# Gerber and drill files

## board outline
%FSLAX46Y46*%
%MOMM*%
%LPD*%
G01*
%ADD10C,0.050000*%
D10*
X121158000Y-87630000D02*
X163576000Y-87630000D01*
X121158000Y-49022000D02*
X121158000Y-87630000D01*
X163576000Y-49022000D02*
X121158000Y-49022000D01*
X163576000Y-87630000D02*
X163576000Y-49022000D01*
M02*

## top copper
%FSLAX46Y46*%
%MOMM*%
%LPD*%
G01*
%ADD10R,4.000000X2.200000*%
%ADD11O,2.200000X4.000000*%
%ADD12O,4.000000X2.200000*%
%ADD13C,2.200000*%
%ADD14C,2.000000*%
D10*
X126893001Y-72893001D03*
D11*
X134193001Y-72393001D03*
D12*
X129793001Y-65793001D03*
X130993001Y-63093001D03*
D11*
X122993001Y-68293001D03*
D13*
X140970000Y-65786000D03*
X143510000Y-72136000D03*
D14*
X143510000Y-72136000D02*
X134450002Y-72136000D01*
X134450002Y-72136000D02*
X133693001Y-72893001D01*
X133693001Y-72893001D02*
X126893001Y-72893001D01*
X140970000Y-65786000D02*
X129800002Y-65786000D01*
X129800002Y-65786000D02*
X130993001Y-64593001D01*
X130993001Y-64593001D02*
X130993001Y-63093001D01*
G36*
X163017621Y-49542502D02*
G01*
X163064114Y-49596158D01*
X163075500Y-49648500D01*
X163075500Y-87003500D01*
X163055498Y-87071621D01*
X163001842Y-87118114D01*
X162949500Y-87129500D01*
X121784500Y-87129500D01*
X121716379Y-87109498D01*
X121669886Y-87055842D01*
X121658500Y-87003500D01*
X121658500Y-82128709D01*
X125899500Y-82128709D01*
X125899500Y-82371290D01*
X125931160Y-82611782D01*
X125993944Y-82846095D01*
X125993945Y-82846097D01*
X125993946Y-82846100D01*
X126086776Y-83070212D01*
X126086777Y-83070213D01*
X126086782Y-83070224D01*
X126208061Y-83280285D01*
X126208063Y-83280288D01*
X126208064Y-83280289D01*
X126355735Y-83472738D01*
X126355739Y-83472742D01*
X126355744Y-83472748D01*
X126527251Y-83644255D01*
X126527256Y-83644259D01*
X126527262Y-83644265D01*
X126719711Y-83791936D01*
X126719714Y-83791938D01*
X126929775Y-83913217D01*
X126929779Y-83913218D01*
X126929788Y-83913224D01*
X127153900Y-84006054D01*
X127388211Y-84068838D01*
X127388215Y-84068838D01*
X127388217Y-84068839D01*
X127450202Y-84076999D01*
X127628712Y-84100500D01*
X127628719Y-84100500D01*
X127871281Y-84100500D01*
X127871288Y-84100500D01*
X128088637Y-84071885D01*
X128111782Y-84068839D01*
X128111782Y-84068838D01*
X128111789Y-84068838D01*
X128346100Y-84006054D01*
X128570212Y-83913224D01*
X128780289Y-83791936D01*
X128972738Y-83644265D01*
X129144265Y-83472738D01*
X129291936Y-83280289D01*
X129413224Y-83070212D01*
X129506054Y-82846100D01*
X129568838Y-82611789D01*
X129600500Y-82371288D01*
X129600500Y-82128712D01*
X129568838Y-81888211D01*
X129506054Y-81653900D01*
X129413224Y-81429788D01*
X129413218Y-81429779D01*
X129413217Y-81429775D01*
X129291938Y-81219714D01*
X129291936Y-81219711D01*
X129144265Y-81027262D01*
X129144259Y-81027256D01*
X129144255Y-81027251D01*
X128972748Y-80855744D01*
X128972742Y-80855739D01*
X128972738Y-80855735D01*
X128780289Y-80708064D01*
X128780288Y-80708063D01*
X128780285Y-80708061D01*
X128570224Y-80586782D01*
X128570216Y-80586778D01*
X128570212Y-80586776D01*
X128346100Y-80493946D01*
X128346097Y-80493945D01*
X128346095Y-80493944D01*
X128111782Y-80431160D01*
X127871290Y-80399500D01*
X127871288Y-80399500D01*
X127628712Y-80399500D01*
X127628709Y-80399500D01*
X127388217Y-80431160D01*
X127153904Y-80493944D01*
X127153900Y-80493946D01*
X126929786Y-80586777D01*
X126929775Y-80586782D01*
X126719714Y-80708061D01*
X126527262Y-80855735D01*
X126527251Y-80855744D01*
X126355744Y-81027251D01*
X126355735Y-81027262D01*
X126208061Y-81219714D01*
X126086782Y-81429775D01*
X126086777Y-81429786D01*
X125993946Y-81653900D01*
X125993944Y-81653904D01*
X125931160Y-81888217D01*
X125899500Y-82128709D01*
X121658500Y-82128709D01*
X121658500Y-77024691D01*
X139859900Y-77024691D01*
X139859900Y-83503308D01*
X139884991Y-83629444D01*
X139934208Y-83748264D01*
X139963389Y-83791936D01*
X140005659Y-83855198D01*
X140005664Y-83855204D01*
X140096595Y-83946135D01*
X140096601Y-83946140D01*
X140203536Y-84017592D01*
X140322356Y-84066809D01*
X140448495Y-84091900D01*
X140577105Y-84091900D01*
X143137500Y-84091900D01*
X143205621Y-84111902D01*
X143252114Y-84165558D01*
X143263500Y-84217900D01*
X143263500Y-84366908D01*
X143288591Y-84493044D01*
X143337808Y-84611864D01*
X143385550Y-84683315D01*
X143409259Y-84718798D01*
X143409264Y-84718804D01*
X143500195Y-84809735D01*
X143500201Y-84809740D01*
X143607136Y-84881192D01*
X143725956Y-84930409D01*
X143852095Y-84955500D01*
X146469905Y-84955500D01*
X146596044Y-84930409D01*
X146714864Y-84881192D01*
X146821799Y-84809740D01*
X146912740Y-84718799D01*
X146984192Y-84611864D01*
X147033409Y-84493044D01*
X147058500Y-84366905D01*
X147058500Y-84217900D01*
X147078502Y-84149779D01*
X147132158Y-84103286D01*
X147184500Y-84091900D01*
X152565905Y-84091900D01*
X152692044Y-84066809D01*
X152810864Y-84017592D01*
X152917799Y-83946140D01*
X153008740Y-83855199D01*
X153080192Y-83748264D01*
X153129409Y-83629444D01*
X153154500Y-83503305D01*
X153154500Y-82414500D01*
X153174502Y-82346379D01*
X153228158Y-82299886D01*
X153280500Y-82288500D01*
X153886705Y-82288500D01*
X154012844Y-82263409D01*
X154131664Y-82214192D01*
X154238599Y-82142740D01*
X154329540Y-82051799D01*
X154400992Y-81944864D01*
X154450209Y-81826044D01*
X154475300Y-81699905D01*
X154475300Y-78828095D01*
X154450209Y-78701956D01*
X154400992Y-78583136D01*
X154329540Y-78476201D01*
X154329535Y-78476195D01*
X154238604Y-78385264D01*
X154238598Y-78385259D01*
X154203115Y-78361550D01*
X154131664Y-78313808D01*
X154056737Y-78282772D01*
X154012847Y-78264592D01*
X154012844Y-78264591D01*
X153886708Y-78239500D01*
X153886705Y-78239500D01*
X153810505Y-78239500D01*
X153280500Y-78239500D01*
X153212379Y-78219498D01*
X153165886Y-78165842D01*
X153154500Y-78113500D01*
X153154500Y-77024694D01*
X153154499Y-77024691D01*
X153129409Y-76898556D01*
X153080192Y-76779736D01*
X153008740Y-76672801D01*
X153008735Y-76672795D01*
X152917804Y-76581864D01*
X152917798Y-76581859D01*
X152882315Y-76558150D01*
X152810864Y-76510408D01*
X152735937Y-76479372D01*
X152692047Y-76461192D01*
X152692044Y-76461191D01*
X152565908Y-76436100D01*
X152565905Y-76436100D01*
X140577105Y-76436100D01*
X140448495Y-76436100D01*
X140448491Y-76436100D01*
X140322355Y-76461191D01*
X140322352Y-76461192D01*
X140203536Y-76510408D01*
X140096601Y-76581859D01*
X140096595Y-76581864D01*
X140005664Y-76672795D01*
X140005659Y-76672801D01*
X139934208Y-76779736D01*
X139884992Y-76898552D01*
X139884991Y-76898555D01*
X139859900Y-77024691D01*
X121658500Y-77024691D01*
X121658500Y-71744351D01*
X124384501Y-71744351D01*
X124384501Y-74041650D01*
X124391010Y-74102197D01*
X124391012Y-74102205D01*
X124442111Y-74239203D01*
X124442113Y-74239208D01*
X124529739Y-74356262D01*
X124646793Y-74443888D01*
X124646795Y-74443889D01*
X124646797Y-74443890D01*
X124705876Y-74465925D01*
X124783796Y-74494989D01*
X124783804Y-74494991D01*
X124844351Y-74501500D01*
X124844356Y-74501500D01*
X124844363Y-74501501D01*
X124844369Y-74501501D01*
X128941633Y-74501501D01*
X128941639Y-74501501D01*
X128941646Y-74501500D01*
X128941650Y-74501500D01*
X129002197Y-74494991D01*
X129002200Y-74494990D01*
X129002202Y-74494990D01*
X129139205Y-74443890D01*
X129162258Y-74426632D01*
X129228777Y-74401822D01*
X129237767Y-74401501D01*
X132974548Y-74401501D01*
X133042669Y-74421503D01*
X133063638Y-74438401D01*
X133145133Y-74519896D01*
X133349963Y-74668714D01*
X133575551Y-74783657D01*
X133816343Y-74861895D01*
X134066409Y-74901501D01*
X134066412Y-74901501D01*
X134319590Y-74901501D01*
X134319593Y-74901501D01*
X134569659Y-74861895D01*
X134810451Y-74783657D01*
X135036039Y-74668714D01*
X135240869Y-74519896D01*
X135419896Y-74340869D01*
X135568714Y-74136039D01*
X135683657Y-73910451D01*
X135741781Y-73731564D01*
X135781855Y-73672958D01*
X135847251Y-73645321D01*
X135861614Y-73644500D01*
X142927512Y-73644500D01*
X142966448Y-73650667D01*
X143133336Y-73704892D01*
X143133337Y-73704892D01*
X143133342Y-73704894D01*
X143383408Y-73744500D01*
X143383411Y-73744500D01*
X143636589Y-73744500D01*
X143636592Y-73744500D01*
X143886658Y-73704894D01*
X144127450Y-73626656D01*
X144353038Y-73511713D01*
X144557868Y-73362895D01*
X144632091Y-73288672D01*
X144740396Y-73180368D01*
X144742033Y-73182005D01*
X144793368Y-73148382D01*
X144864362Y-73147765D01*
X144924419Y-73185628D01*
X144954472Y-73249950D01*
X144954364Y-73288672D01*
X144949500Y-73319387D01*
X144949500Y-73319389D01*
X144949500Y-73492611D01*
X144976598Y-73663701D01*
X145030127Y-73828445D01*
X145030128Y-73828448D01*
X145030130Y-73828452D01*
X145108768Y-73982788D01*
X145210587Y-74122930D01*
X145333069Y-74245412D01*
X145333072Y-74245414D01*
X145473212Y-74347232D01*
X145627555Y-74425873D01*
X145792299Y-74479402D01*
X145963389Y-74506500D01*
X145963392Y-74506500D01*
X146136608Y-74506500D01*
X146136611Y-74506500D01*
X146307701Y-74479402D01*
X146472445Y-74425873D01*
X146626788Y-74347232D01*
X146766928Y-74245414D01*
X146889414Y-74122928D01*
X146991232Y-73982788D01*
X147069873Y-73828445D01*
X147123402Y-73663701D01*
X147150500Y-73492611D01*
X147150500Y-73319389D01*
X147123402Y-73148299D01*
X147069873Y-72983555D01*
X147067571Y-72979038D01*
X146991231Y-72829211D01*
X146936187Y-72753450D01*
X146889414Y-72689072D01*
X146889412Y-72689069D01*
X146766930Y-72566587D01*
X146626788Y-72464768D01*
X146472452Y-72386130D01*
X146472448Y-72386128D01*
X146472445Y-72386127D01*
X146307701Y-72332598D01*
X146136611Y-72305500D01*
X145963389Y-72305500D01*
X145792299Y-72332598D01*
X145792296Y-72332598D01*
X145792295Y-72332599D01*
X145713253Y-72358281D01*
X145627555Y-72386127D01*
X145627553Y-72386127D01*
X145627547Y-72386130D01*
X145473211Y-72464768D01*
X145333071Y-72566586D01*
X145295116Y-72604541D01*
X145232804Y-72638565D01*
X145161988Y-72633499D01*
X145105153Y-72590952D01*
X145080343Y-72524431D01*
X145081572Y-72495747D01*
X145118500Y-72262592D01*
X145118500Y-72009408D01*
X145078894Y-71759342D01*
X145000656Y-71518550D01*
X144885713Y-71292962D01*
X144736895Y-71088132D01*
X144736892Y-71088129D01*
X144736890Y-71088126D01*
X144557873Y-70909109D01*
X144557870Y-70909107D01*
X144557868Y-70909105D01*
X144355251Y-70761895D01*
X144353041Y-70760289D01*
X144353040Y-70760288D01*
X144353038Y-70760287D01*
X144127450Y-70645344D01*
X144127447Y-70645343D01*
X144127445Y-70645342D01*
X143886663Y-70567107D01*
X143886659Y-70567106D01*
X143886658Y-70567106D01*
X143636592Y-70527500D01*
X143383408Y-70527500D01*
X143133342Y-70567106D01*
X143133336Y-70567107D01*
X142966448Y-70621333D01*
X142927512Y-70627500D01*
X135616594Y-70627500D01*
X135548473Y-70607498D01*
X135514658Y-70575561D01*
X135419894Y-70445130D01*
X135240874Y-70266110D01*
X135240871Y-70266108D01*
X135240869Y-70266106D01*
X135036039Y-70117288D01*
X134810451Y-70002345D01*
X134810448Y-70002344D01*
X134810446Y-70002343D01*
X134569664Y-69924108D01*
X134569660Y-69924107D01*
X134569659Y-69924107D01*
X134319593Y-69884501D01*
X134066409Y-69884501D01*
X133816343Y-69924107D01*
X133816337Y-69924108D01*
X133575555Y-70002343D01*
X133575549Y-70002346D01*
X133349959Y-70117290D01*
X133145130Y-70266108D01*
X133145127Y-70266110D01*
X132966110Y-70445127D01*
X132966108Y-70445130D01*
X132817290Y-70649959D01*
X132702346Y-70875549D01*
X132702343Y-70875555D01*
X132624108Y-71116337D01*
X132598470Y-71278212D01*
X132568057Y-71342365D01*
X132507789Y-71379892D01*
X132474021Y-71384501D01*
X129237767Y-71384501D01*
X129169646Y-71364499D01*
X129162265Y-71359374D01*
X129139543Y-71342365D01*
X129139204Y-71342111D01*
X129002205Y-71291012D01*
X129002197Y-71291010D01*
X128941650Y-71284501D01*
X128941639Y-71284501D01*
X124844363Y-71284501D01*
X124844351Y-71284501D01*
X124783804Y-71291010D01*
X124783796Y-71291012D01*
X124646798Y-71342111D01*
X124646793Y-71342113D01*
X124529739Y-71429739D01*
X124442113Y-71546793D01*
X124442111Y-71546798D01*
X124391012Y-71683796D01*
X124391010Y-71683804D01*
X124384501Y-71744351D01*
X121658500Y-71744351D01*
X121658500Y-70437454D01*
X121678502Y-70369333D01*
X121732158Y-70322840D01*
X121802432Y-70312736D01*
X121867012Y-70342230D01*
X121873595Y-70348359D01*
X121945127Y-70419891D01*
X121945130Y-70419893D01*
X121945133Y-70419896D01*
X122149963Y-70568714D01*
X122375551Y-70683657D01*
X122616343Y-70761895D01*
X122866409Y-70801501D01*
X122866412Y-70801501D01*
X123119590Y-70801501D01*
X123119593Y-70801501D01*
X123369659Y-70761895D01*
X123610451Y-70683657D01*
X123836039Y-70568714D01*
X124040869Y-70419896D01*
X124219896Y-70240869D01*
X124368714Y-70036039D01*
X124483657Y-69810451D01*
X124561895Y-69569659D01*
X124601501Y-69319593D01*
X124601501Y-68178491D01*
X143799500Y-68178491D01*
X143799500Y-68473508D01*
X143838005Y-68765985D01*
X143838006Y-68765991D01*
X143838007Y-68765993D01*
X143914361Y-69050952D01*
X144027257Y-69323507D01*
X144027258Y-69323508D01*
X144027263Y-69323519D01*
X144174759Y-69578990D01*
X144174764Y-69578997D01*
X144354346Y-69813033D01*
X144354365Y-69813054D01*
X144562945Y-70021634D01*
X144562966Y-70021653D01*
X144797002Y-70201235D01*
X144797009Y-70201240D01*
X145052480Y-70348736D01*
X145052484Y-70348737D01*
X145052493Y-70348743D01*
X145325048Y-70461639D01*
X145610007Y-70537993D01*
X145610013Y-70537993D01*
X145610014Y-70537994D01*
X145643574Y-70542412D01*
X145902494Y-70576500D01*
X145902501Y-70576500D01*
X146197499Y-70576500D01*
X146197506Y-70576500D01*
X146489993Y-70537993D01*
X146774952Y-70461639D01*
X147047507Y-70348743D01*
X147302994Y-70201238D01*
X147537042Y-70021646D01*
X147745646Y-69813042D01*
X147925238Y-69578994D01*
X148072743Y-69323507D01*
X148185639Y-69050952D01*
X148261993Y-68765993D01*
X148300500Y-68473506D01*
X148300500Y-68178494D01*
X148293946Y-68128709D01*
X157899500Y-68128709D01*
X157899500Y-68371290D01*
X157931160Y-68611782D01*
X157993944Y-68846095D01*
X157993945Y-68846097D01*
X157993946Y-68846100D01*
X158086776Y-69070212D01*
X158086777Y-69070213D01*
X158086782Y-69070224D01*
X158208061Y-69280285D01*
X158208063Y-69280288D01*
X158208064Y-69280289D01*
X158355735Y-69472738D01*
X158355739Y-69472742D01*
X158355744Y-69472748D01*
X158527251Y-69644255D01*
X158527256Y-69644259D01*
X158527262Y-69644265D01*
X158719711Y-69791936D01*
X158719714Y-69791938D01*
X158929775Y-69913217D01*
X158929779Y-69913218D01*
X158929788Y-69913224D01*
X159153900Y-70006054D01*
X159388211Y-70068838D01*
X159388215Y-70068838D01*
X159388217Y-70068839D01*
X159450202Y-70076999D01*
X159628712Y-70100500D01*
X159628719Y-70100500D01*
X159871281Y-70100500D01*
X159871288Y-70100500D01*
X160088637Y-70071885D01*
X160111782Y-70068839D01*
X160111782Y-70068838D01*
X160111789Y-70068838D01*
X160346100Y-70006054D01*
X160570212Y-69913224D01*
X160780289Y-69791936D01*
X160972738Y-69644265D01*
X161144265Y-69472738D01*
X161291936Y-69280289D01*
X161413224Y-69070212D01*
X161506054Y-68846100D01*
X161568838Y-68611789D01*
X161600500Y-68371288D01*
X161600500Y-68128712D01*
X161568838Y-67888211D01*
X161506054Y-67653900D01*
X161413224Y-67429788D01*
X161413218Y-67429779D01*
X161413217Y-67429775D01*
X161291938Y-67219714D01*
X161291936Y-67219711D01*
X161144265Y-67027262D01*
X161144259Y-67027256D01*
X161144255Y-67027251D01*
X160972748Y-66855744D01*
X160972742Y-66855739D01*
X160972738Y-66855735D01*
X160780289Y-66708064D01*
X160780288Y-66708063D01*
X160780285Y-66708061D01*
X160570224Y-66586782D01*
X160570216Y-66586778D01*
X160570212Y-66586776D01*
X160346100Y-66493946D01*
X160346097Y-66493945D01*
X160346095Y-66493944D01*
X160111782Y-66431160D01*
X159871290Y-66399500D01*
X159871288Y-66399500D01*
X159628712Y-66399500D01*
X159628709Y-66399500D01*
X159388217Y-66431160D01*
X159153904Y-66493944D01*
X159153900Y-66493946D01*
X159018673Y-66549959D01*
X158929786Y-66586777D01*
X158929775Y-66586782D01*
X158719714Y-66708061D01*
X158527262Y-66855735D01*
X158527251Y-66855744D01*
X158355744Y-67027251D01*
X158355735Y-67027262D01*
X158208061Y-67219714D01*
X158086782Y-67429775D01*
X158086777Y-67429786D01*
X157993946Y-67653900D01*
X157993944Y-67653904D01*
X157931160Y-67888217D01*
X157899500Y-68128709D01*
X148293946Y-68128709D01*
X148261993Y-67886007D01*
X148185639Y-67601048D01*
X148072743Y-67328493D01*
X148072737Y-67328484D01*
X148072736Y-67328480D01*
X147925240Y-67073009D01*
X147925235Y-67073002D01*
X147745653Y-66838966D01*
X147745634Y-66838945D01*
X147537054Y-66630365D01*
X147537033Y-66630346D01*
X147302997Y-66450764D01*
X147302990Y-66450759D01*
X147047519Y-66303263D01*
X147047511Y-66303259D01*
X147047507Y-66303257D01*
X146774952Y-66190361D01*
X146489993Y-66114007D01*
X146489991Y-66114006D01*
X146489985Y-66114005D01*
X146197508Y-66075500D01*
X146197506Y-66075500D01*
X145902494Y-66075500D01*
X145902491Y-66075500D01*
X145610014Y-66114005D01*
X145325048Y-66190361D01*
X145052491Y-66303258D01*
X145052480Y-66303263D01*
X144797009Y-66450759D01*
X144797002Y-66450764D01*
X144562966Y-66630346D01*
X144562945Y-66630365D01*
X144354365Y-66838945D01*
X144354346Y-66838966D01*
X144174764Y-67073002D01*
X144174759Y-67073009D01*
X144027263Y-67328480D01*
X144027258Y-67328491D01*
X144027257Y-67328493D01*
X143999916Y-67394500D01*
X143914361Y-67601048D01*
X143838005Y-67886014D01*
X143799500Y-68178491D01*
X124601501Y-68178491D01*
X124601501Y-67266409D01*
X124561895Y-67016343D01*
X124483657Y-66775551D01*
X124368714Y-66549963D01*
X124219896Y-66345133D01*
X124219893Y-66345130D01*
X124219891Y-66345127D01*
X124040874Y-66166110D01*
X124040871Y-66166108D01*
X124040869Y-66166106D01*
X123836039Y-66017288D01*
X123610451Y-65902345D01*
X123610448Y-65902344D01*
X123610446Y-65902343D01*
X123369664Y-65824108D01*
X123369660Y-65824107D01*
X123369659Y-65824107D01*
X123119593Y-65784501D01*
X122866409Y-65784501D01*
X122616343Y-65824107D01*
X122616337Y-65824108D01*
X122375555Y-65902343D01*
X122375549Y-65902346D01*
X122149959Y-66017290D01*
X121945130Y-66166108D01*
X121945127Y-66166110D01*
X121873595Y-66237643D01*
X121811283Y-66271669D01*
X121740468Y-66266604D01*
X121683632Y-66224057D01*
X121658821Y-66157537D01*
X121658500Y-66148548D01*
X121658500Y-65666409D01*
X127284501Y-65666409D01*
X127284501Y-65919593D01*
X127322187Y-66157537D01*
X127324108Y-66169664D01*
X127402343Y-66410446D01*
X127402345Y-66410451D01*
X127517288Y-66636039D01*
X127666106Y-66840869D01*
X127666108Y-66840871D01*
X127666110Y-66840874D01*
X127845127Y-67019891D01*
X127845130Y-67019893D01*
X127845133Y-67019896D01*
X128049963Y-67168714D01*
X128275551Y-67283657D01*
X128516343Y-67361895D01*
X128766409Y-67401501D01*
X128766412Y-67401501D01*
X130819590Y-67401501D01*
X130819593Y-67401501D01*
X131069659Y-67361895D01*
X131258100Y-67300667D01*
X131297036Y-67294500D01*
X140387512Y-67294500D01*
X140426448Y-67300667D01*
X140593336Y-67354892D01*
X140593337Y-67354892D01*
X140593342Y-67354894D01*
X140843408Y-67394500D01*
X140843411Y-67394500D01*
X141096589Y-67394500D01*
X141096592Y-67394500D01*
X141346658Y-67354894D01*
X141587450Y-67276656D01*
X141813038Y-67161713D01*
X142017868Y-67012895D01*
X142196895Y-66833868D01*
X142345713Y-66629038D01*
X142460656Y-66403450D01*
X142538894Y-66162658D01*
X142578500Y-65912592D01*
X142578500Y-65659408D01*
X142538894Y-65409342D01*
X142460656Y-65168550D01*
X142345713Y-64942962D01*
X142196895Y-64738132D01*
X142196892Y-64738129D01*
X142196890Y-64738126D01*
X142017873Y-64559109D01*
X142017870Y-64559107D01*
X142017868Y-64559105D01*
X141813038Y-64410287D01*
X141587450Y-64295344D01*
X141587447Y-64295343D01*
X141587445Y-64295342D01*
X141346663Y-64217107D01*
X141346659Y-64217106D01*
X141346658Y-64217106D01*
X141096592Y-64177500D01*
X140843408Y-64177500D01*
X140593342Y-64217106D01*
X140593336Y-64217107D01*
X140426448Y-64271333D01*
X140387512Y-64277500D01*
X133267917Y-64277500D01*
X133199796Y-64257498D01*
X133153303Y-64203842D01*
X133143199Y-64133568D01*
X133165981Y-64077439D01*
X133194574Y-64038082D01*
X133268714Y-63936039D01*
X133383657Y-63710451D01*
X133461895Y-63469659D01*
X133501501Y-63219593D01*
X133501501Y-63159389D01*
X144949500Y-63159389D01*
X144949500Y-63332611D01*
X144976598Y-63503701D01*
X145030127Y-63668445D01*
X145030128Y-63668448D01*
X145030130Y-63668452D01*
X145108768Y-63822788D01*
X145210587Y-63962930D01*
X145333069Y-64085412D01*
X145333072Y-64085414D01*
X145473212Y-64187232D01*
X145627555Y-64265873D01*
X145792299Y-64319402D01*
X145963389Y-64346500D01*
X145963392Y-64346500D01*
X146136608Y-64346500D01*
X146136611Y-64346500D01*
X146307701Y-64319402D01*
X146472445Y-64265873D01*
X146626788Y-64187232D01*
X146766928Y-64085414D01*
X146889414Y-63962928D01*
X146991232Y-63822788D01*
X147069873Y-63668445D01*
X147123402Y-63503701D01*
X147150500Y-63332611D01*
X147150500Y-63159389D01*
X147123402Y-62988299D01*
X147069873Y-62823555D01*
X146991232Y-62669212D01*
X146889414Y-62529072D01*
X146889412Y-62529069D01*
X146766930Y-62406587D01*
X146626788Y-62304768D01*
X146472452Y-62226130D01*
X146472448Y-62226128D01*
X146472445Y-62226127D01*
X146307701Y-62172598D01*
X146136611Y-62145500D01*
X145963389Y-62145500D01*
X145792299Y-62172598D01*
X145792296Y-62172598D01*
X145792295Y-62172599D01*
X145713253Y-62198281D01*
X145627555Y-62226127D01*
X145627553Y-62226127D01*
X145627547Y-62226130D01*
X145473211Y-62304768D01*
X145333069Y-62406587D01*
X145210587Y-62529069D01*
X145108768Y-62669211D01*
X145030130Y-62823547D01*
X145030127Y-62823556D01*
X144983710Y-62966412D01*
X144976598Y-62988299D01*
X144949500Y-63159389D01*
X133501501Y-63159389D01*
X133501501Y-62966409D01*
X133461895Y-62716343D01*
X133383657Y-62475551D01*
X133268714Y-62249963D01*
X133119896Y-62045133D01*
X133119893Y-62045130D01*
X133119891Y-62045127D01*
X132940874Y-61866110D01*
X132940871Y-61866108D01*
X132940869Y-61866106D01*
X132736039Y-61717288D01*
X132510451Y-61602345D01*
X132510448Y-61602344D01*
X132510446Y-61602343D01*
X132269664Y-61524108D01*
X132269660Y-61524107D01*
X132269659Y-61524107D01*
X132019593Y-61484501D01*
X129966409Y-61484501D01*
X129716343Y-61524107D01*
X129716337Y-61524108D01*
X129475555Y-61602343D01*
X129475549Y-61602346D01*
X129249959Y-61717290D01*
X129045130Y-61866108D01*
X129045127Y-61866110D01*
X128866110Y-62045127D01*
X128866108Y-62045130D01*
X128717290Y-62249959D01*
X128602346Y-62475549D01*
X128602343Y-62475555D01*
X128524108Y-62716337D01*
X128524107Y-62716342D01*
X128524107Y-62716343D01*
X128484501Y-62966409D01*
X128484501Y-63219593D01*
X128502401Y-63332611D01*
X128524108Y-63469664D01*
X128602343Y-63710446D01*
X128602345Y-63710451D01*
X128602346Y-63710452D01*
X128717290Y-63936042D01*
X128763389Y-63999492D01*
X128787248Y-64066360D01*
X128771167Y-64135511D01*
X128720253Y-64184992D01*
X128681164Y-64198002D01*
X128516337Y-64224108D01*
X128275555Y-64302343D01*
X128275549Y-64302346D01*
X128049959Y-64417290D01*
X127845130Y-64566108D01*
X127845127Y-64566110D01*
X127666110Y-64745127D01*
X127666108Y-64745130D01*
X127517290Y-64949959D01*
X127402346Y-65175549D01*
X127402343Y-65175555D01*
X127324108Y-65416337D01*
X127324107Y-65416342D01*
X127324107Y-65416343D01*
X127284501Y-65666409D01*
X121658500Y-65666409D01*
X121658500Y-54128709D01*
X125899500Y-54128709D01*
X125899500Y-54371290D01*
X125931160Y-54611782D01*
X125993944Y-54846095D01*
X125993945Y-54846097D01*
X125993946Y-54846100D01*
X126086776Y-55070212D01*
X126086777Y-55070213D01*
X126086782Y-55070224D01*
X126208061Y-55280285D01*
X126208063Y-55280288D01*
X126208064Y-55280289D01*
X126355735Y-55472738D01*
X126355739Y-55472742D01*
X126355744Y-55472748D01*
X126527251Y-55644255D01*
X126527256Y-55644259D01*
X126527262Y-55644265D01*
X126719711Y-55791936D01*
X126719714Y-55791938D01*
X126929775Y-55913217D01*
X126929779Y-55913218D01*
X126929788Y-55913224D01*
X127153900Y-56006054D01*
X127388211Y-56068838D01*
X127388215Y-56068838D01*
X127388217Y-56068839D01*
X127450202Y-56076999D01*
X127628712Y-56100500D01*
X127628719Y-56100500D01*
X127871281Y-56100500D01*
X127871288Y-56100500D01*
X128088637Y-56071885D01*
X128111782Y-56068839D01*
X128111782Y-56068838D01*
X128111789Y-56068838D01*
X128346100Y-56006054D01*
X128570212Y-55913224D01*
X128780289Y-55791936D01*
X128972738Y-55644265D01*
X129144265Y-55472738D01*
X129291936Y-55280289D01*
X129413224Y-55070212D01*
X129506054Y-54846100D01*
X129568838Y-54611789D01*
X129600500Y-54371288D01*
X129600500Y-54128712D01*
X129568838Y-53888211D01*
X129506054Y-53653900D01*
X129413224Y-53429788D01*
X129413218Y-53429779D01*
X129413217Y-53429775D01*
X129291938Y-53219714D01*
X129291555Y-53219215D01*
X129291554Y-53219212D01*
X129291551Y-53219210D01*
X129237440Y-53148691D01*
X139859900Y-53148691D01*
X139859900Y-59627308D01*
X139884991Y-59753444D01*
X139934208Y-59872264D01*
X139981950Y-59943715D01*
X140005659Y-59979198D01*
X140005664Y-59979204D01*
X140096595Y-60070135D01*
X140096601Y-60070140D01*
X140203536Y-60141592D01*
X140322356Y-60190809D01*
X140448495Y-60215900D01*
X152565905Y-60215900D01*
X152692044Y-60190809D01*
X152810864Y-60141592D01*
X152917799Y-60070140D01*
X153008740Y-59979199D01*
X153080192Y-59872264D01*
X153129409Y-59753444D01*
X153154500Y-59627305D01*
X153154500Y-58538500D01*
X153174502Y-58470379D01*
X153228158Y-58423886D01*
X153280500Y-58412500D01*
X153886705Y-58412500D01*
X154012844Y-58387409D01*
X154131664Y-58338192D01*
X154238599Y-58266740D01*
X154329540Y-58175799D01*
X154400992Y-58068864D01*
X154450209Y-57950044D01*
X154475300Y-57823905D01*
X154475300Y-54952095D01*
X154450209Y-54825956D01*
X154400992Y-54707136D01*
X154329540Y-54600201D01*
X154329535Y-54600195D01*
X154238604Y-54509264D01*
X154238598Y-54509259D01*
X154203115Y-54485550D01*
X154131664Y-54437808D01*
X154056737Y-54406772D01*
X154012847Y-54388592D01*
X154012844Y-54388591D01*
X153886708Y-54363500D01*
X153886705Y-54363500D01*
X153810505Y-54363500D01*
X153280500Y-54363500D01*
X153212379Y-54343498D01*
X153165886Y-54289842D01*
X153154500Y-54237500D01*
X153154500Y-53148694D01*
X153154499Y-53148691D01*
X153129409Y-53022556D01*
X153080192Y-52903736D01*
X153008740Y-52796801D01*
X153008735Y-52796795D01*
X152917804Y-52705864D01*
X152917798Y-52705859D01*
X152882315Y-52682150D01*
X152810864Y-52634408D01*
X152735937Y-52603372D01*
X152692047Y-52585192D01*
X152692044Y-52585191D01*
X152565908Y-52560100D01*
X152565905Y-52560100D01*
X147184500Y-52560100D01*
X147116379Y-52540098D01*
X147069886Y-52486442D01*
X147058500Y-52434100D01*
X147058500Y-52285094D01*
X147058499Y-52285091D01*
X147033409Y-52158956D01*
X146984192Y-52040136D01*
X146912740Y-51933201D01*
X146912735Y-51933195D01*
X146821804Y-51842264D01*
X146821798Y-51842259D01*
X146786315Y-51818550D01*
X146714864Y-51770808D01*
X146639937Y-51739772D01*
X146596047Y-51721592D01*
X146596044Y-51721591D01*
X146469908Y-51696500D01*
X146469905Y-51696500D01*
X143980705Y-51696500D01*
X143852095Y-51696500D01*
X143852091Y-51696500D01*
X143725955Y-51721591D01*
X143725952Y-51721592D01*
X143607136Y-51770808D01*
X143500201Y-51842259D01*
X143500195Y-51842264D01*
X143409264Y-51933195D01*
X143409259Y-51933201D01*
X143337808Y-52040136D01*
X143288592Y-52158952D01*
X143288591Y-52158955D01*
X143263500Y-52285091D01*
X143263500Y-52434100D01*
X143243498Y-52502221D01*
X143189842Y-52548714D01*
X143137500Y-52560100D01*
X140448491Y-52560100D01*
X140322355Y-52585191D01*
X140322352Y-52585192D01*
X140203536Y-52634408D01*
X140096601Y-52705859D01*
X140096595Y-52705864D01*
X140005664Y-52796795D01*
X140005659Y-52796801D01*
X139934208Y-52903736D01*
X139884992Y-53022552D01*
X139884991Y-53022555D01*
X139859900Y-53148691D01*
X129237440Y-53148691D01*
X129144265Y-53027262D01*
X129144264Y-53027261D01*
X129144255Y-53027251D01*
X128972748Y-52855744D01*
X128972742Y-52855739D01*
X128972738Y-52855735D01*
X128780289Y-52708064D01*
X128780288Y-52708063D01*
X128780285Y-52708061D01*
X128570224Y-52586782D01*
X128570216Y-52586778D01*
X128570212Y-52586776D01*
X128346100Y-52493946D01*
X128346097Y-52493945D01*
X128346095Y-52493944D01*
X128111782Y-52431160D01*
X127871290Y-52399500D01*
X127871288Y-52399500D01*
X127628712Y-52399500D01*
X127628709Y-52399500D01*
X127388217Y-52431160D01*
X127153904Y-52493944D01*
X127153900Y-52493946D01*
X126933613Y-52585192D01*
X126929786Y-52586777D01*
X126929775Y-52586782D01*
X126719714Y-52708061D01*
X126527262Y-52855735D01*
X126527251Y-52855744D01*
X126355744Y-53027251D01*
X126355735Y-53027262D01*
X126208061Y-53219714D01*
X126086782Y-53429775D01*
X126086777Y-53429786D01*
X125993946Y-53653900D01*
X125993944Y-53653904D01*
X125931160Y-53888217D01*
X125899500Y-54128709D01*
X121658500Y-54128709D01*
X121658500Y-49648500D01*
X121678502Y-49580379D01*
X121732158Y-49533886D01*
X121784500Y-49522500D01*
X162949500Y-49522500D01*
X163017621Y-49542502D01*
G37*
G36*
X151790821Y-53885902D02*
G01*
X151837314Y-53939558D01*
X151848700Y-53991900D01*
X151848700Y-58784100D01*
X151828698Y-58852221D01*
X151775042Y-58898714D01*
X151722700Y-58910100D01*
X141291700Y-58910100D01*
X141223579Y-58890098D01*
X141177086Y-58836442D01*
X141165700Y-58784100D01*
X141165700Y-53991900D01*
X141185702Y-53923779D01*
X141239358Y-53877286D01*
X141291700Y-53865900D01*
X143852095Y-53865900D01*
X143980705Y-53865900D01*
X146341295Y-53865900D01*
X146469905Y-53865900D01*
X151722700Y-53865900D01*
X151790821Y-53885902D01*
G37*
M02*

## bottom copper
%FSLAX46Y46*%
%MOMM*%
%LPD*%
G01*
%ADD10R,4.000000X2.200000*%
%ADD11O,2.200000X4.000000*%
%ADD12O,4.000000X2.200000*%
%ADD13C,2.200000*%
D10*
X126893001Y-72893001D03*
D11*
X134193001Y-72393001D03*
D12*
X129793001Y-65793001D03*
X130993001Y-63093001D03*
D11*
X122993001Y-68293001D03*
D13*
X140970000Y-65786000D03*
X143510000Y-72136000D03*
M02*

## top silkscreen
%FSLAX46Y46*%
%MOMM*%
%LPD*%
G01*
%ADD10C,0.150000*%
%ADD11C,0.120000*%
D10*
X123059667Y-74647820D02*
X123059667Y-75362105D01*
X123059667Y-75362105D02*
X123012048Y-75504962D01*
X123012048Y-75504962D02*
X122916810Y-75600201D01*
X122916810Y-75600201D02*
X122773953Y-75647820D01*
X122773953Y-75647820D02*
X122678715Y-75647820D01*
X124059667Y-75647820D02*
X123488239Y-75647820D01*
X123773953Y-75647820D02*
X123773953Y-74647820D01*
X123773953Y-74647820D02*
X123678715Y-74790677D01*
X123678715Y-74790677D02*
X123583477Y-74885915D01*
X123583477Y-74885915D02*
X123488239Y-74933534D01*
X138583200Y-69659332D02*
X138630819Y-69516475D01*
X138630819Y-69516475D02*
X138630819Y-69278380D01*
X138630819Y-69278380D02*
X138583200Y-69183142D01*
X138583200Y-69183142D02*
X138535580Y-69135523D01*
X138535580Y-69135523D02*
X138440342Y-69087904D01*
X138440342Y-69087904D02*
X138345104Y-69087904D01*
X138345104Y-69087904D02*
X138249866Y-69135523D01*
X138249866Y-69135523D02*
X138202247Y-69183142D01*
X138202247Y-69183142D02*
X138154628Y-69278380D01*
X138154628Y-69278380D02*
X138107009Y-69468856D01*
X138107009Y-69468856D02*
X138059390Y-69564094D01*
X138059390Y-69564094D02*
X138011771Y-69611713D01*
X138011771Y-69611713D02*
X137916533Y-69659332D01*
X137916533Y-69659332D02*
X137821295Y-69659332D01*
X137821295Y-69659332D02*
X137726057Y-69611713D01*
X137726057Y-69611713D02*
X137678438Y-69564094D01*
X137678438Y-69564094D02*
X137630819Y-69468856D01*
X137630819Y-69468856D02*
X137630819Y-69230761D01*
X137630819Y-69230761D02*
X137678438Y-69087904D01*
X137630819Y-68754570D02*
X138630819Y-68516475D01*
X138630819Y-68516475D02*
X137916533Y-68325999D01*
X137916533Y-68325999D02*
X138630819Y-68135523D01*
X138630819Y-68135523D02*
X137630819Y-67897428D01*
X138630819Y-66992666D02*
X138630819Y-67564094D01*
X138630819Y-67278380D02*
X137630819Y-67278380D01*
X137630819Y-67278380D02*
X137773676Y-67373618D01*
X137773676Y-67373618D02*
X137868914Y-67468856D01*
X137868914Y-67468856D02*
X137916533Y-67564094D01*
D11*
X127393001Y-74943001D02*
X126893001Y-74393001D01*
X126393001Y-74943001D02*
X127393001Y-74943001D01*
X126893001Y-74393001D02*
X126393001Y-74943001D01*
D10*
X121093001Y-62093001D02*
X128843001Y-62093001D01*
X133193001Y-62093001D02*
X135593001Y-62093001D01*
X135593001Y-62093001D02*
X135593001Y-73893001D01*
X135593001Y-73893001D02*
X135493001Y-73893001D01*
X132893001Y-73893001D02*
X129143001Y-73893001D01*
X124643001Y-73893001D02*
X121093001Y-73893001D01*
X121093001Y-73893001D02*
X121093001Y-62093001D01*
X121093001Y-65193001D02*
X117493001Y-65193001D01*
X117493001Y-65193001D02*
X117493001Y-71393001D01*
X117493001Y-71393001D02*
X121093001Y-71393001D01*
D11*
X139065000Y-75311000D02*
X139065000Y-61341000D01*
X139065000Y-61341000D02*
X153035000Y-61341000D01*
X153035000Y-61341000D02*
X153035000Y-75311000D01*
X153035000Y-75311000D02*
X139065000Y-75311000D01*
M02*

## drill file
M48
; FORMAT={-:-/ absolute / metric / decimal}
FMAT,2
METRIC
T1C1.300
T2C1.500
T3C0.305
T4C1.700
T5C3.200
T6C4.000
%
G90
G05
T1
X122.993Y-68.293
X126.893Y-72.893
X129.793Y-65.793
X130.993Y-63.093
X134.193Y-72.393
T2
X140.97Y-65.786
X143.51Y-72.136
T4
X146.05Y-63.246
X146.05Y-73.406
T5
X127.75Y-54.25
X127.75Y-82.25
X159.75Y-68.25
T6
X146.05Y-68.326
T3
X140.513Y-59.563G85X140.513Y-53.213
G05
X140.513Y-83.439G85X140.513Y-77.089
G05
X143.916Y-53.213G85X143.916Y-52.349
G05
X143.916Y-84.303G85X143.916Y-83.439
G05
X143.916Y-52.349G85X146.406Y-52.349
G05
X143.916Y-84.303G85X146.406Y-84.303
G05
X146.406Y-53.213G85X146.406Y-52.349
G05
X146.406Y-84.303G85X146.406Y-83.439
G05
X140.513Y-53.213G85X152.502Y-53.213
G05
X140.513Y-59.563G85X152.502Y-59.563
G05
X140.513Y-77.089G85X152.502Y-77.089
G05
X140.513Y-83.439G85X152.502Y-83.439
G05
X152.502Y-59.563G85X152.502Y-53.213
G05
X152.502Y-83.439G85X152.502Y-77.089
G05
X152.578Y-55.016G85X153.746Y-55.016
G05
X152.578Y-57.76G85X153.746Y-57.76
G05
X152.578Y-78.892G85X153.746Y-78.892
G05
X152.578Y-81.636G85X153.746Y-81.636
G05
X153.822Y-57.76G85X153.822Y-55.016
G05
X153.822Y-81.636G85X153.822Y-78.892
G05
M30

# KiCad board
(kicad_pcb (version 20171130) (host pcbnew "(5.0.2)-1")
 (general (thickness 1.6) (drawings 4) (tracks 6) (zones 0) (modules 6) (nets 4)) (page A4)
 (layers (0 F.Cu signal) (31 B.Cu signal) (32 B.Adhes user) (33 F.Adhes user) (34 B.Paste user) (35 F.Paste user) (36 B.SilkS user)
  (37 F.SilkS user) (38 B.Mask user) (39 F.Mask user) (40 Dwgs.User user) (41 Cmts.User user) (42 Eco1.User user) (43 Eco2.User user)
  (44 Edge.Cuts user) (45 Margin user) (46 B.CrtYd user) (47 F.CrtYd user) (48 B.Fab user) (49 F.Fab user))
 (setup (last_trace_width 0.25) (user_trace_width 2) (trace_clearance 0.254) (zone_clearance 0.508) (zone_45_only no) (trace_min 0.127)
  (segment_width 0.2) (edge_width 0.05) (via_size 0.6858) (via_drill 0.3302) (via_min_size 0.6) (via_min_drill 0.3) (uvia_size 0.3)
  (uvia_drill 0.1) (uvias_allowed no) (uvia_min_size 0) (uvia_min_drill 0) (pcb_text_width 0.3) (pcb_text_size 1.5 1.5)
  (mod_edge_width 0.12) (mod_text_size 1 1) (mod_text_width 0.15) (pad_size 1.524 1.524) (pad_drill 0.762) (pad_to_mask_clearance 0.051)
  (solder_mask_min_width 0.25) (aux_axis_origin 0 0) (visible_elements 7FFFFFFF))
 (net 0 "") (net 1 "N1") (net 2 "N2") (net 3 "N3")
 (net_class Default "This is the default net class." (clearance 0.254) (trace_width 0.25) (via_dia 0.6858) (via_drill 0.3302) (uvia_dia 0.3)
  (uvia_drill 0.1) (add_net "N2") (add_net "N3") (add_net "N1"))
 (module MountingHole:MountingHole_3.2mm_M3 (layer F.Cu) (at 159.75 68.25)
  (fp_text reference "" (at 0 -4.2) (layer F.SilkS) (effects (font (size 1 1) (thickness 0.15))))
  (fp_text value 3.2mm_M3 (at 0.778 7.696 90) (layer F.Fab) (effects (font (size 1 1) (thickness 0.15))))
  (pad 1 np_thru_hole circle (at 0 0) (size 3.2 3.2) (drill 3.2) (layers *.Cu *.Mask)))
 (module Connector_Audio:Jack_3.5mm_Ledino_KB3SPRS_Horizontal (layer F.Cu) (at 126.893001 72.893001)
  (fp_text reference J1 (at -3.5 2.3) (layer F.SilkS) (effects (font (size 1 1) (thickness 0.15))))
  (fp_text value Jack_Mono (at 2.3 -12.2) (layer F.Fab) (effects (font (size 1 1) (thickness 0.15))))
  (fp_line (start 0.5 2.05) (end 0 1.5) (layer F.SilkS) (width 0.12))
  (fp_line (start -0.5 2.05) (end 0.5 2.05) (layer F.SilkS) (width 0.12))
  (fp_line (start 0 1.5) (end -0.5 2.05) (layer F.SilkS) (width 0.12))
  (fp_line (start -5.8 -10.8) (end 1.95 -10.8) (layer F.SilkS) (width 0.15))
  (fp_line (start 6.3 -10.8) (end 8.7 -10.8) (layer F.SilkS) (width 0.15))
  (fp_line (start 8.7 -10.8) (end 8.7 1) (layer F.SilkS) (width 0.15))
  (fp_line (start 8.7 1) (end 8.6 1) (layer F.SilkS) (width 0.15))
  (fp_line (start 6 1) (end 2.25 1) (layer F.SilkS) (width 0.15))
  (fp_line (start -2.25 1) (end -5.8 1) (layer F.SilkS) (width 0.15))
  (fp_line (start -5.8 1) (end -5.8 -10.8) (layer F.SilkS) (width 0.15))
  (fp_line (start -5.8 -7.7) (end -9.4 -7.7) (layer F.SilkS) (width 0.15))
  (fp_line (start -9.4 -7.7) (end -9.4 -1.5) (layer F.SilkS) (width 0.15))
  (fp_line (start -9.4 -1.5) (end -5.8 -1.5) (layer F.SilkS) (width 0.15))
  (pad T thru_hole rect (at 0 0) (size 4 2.2) (drill 1.3) (layers *.Cu *.Mask) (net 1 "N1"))
  (pad TN thru_hole oval (at 7.3 -0.5 90) (size 4 2.2) (drill 1.3) (layers *.Cu *.Mask) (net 1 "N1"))
  (pad RN thru_hole oval (at 2.9 -7.1) (size 4 2.2) (drill 1.3) (layers *.Cu *.Mask) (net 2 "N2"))
  (pad R thru_hole oval (at 4.1 -9.8) (size 4 2.2) (drill 1.3) (layers *.Cu *.Mask) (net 2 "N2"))
  (pad S thru_hole oval (at -3.9 -4.6) (size 2.2 4) (drill 1.3) (layers *.Cu *.Mask) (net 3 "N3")))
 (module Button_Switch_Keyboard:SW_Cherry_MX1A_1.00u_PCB (layer F.Cu) (at 140.97 65.786 90)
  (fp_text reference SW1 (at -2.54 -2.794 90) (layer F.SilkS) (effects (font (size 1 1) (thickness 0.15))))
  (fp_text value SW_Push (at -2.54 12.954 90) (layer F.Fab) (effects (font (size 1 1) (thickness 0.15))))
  (fp_line (start -9.525 -1.905) (end 4.445 -1.905) (layer F.SilkS) (width 0.12))
  (fp_line (start 4.445 -1.905) (end 4.445 12.065) (layer F.SilkS) (width 0.12))
  (fp_line (start 4.445 12.065) (end -9.525 12.065) (layer F.SilkS) (width 0.12))
  (fp_line (start -9.525 12.065) (end -9.525 -1.905) (layer F.SilkS) (width 0.12))
  (pad 1 thru_hole circle (at 0 0 90) (size 2.2 2.2) (drill 1.5) (layers *.Cu *.Mask) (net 2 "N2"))
  (pad 2 thru_hole circle (at -6.35 2.54 90) (size 2.2 2.2) (drill 1.5) (layers *.Cu *.Mask) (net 1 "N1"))
  (pad "" np_thru_hole circle (at -2.54 5.08 90) (size 4 4) (drill 4) (layers *.Cu *.Mask))
  (pad "" np_thru_hole circle (at -7.62 5.08 90) (size 1.7 1.7) (drill 1.7) (layers *.Cu *.Mask))
  (pad "" np_thru_hole circle (at 2.54 5.08 90) (size 1.7 1.7) (drill 1.7) (layers *.Cu *.Mask)))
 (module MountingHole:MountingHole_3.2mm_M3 (layer F.Cu) (at 127.75 54.25)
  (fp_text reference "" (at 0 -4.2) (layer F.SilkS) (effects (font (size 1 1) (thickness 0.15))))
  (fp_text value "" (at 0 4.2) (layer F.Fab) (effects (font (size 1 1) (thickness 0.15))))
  (pad 1 np_thru_hole circle (at 0 0) (size 3.2 3.2) (drill 3.2) (layers *.Cu *.Mask)))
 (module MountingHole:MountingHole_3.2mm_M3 (layer F.Cu) (at 127.75 82.25)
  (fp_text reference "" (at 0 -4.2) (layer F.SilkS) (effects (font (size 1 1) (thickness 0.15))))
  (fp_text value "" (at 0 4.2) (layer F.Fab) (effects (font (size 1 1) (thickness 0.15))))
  (pad 1 np_thru_hole circle (at 0 0) (size 3.2 3.2) (drill 3.2) (layers *.Cu *.Mask)))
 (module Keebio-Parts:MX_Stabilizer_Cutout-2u (layer F.Cu) (at 146.05 68.326 90)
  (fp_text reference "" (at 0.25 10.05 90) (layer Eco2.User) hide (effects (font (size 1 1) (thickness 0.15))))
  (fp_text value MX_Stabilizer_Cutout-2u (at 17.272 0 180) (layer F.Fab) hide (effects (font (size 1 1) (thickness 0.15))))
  (pad "" np_thru_hole oval (at -11.938 7.7724 90) (size 3.048 0.3048) (drill oval 3.048 0.3048) (layers *.Cu *.Mask))
  (pad "" np_thru_hole oval (at -10.5664 7.112 90) (size 0.3048 1.4732) (drill oval 0.3048 1.4732) (layers *.Cu *.Mask))
  (pad "" np_thru_hole oval (at -13.3096 7.112 90) (size 0.3048 1.4732) (drill oval 0.3048 1.4732) (layers *.Cu *.Mask))
  (pad "" np_thru_hole oval (at -15.5448 0.3556 90) (size 1.1684 0.3048) (drill oval 1.1684 0.3048) (layers *.Cu *.Mask))
  (pad "" np_thru_hole oval (at -11.938 6.4516 90) (size 6.6548 0.3048) (drill oval 6.6548 0.3048) (layers *.Cu *.Mask))
  (pad "" np_thru_hole oval (at -8.763 0.4572 90) (size 0.3048 12.2936) (drill oval 0.3048 12.2936) (layers *.Cu *.Mask))
  (pad "" np_thru_hole oval (at -15.113 0.4572 90) (size 0.3048 12.2936) (drill oval 0.3048 12.2936) (layers *.Cu *.Mask))
  (pad "" np_thru_hole oval (at -15.9766 -0.889 90) (size 0.3048 2.794) (drill oval 0.3048 2.794) (layers *.Cu *.Mask))
  (pad "" np_thru_hole oval (at -15.5448 -2.1336 90) (size 1.1684 0.3048) (drill oval 1.1684 0.3048) (layers *.Cu *.Mask))
  (pad "" np_thru_hole oval (at -11.938 -5.5372 90) (size 6.6548 0.3048) (drill oval 6.6548 0.3048) (layers *.Cu *.Mask))
  (pad "" np_thru_hole oval (at 15.5448 0.3556 90) (size 1.1684 0.3048) (drill oval 1.1684 0.3048) (layers *.Cu *.Mask))
  (pad "" np_thru_hole oval (at 13.3096 7.112 90) (size 0.3048 1.4732) (drill oval 0.3048 1.4732) (layers *.Cu *.Mask))
  (pad "" np_thru_hole oval (at 15.5448 -2.1336 90) (size 1.1684 0.3048) (drill oval 1.1684 0.3048) (layers *.Cu *.Mask))
  (pad "" np_thru_hole oval (at 10.5664 7.112 90) (size 0.3048 1.4732) (drill oval 0.3048 1.4732) (layers *.Cu *.Mask))
  (pad "" np_thru_hole oval (at 15.9766 -0.889 90) (size 0.3048 2.794) (drill oval 0.3048 2.794) (layers *.Cu *.Mask))
  (pad "" np_thru_hole oval (at 15.113 0.4572 90) (size 0.3048 12.2936) (drill oval 0.3048 12.2936) (layers *.Cu *.Mask))
  (pad "" np_thru_hole oval (at 11.938 6.4516 90) (size 6.6548 0.3048) (drill oval 6.6548 0.3048) (layers *.Cu *.Mask))
  (pad "" np_thru_hole oval (at 8.763 0.4572 90) (size 0.3048 12.2936) (drill oval 0.3048 12.2936) (layers *.Cu *.Mask))
  (pad "" np_thru_hole oval (at 11.938 -5.5372 90) (size 6.6548 0.3048) (drill oval 6.6548 0.3048) (layers *.Cu *.Mask))
  (pad "" np_thru_hole oval (at 11.938 7.7724 90) (size 3.048 0.3048) (drill oval 3.048 0.3048) (layers *.Cu *.Mask)))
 (gr_line (start 121.158 87.63) (end 163.576 87.63) (angle 90) (layer Edge.Cuts) (width 0.05))
 (gr_line (start 121.158 49.022) (end 121.158 87.63) (angle 90) (layer Edge.Cuts) (width 0.05))
 (gr_line (start 163.576 49.022) (end 121.158 49.022) (angle 90) (layer Edge.Cuts) (width 0.05))
 (gr_line (start 163.576 87.63) (end 163.576 49.022) (angle 90) (layer Edge.Cuts) (width 0.05))
 (segment (start 143.51 72.136) (end 134.450002 72.136) (width 2) (layer F.Cu) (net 1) (status C00000))
 (segment (start 134.450002 72.136) (end 133.693001 72.893001) (width 2) (layer F.Cu) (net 1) (status C00000))
 (segment (start 133.693001 72.893001) (end 126.893001 72.893001) (width 2) (layer F.Cu) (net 1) (status C00000))
 (segment (start 140.97 65.786) (end 129.800002 65.786) (width 2) (layer F.Cu) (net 2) (status C00000))
 (segment (start 129.800002 65.786) (end 130.993001 64.593001) (width 2) (layer F.Cu) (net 2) (status 400000))
 (segment (start 130.993001 64.593001) (end 130.993001 63.093001) (width 2) (layer F.Cu) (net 2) (status 800000))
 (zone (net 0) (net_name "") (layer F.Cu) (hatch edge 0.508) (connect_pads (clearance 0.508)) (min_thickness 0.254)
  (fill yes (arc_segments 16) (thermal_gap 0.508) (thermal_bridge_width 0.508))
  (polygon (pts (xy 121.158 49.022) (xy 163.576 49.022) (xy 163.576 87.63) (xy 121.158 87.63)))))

